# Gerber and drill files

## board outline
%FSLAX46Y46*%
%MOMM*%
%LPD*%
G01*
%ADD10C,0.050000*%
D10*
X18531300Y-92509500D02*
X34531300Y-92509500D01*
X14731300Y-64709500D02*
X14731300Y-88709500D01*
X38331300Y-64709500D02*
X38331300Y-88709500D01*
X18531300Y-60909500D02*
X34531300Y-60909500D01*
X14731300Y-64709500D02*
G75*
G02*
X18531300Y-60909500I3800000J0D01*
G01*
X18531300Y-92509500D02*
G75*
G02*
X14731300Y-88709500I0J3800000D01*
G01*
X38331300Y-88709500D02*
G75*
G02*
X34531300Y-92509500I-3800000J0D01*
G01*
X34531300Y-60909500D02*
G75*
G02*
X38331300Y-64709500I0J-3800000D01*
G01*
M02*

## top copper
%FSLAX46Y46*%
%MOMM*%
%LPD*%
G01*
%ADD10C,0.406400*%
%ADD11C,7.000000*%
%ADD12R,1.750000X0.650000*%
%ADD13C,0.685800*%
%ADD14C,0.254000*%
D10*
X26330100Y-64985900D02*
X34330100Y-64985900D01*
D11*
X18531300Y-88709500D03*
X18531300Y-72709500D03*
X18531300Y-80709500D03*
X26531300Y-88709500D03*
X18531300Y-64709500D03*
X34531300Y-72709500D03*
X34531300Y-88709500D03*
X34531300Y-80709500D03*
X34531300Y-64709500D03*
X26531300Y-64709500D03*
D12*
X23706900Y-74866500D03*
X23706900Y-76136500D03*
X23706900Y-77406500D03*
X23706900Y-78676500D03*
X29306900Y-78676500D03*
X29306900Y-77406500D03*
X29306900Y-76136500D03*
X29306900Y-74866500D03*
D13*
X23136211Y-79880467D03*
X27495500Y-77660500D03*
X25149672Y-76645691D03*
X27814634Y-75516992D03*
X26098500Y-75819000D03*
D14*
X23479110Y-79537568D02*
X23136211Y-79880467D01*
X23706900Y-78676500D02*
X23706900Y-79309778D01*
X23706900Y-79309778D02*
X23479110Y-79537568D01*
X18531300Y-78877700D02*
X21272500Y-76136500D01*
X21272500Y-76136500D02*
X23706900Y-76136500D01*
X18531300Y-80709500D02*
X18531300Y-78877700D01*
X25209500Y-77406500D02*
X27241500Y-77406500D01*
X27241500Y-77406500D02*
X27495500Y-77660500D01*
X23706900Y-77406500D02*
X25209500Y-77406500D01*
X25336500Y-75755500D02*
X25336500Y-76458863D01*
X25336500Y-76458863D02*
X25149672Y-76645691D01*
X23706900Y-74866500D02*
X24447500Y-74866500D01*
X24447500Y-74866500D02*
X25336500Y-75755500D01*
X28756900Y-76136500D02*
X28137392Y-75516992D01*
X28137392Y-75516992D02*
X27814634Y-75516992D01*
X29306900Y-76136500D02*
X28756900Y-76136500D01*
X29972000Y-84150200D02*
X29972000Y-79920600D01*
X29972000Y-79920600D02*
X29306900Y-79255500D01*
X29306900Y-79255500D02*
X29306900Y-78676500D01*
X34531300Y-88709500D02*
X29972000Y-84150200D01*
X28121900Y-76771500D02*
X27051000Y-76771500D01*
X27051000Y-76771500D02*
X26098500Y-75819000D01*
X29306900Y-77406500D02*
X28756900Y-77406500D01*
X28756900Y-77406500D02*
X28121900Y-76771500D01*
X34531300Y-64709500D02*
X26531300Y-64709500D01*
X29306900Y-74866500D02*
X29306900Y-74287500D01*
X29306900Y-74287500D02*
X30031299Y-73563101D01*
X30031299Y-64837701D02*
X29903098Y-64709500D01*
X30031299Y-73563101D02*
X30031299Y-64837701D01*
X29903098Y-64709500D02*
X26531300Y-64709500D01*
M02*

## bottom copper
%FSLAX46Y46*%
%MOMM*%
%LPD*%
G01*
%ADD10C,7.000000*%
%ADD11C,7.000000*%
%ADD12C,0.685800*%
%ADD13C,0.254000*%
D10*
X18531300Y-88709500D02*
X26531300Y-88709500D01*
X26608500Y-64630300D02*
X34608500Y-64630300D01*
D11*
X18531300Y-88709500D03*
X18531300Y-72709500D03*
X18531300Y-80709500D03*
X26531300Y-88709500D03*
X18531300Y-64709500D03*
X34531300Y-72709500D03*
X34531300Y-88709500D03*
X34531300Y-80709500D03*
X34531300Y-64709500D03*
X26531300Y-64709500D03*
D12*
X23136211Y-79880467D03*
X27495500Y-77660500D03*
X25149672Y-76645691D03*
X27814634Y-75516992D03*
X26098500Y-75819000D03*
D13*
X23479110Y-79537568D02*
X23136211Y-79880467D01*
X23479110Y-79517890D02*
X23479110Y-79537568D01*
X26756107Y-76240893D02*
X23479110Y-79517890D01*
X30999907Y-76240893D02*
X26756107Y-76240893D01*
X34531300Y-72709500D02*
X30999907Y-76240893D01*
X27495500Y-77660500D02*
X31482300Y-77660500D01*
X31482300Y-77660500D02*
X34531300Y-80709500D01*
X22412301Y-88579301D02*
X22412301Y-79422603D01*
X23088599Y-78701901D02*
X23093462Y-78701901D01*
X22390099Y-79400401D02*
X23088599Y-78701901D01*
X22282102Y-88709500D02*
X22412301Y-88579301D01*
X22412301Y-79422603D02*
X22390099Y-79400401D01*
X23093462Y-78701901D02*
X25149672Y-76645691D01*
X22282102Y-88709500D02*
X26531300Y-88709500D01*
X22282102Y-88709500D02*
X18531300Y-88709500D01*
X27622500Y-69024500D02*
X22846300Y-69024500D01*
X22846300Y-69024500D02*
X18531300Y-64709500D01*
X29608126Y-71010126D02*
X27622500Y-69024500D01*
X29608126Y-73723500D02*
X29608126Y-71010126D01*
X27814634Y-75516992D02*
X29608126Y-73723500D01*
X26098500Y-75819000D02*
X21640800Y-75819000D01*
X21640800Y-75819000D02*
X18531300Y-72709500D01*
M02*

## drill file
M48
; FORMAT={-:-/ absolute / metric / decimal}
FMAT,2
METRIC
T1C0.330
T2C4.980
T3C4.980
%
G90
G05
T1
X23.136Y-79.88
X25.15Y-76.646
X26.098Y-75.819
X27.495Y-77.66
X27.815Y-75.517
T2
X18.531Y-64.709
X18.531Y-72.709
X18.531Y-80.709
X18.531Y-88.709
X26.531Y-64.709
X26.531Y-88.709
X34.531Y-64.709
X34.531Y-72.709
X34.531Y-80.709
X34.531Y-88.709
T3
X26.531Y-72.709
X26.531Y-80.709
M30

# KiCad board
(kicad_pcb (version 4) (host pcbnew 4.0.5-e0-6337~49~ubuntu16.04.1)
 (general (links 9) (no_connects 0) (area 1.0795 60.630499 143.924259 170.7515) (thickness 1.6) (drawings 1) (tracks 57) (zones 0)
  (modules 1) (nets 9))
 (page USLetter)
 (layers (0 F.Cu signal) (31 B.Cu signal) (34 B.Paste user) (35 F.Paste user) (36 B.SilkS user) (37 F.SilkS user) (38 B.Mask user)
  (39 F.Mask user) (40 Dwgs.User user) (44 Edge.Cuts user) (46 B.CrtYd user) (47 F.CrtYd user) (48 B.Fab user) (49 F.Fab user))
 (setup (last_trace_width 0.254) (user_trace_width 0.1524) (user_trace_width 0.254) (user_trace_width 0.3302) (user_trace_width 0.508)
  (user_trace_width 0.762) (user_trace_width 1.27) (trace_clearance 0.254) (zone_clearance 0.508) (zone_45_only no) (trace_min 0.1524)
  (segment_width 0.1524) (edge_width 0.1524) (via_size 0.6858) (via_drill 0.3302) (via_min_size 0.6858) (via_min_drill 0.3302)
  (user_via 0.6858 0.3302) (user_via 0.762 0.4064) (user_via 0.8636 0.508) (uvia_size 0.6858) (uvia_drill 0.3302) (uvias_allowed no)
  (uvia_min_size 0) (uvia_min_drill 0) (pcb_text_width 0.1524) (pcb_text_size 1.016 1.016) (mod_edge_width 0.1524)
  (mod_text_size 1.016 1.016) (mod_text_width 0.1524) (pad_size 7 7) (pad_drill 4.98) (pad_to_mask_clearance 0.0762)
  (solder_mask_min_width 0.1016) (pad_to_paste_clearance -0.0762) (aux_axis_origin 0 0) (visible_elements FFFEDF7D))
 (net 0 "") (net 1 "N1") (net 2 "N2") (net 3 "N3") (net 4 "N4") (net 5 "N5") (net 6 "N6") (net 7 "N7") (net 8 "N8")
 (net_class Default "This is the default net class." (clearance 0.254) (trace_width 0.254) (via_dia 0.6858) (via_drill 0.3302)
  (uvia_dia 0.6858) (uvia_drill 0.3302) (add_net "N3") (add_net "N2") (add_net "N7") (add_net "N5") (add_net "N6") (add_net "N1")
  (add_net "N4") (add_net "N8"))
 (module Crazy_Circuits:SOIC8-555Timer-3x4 (layer F.Cu) (at 18.5313 88.7095)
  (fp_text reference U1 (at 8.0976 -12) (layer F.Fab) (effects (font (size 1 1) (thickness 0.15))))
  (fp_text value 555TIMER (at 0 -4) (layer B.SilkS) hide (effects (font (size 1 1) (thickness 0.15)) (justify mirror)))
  (fp_line (start 0 0) (end 8 0) (layer B.Cu) (width 7))
  (fp_line (start 0 3.8) (end 16 3.8) (layer Edge.Cuts) (width 0.05))
  (fp_line (start -3.8 -24) (end -3.8 0) (layer Edge.Cuts) (width 0.05))
  (fp_line (start 19.8 -24) (end 19.8 0) (layer Edge.Cuts) (width 0.05))
  (fp_line (start 0 -27.8) (end 16 -27.8) (layer Edge.Cuts) (width 0.05))
  (fp_arc (start 0 -24) (end -3.8 -24) (angle 90) (layer Edge.Cuts) (width 0.05))
  (fp_arc (start 0 0) (end 0 3.8) (angle 90) (layer Edge.Cuts) (width 0.05))
  (fp_arc (start 16 0) (end 19.8 0) (angle 90) (layer Edge.Cuts) (width 0.05))
  (fp_arc (start 16 -24) (end 16 -27.8) (angle 90) (layer Edge.Cuts) (width 0.05))
  (fp_line (start 7.7988 -23.7236) (end 15.7988 -23.7236) (layer F.Cu) (width 0.4064))
  (fp_line (start 8.0772 -24.0792) (end 16.0772 -24.0792) (layer B.Cu) (width 7))
  (pad e thru_hole circle (at 0 0 270) (size 7 7) (drill 4.98) (layers *.Cu *.Mask))
  (pad "" np_thru_hole circle (at 8 -16 270) (size 4.98 4.98) (drill 4.98) (layers *.Cu))
  (pad 6 thru_hole circle (at 0 -16 270) (size 7 7) (drill 4.98) (layers *.Cu B.Mask) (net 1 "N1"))
  (pad 2 thru_hole circle (at 0 -8 270) (size 7 7) (drill 4.98) (layers *.Cu B.Mask) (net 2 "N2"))
  (pad "" np_thru_hole circle (at 8 -8 270) (size 4.98 4.98) (drill 4.98) (layers *.Cu))
  (pad 1 thru_hole circle (at 8 0 270) (size 7 7) (drill 4.98) (layers *.Cu *.Mask) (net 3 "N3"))
  (pad 7 thru_hole circle (at 0 -24 270) (size 7 7) (drill 4.98) (layers *.Cu B.Mask) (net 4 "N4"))
  (pad 4 thru_hole circle (at 16 -16 270) (size 7 7) (drill 4.98) (layers *.Cu B.Mask) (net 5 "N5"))
  (pad 5 thru_hole circle (at 16 0 270) (size 7 7) (drill 4.98) (layers *.Cu B.Mask) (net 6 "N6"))
  (pad 3 thru_hole circle (at 16 -8 270) (size 7 7) (drill 4.98) (layers *.Cu B.Mask) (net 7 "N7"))
  (pad 8 thru_hole circle (at 16 -24 270) (size 7 7) (drill 4.98) (layers *.Cu *.Mask) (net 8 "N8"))
  (pad 8 thru_hole circle (at 8 -24 270) (size 7 7) (drill 4.98) (layers *.Cu *.Mask) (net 8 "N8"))
  (pad 1 smd rect (at 5.1756 -13.843) (size 1.75 0.65) (layers F.Cu F.Paste F.Mask) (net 3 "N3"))
  (pad 2 smd rect (at 5.1756 -12.573) (size 1.75 0.65) (layers F.Cu F.Paste F.Mask) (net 2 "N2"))
  (pad 3 smd rect (at 5.1756 -11.303) (size 1.75 0.65) (layers F.Cu F.Paste F.Mask) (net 7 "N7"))
  (pad 4 smd rect (at 5.1756 -10.033) (size 1.75 0.65) (layers F.Cu F.Paste F.Mask) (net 5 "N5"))
  (pad 5 smd rect (at 10.7756 -10.033) (size 1.75 0.65) (layers F.Cu F.Paste F.Mask) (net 6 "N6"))
  (pad 6 smd rect (at 10.7756 -11.303) (size 1.75 0.65) (layers F.Cu F.Paste F.Mask) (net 1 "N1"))
  (pad 7 smd rect (at 10.7756 -12.573) (size 1.75 0.65) (layers F.Cu F.Paste F.Mask) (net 4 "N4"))
  (pad 8 smd rect (at 10.7756 -13.843) (size 1.75 0.65) (layers F.Cu F.Paste F.Mask) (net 8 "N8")))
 (segment (start 23.47911 79.537568) (end 23.136211 79.880467) (width 0.254) (layer B.Cu) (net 5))
 (segment (start 23.47911 79.51789) (end 23.47911 79.537568) (width 0.254) (layer B.Cu) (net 5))
 (segment (start 26.756107 76.240893) (end 23.47911 79.51789) (width 0.254) (layer B.Cu) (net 5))
 (segment (start 30.999907 76.240893) (end 26.756107 76.240893) (width 0.254) (layer B.Cu) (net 5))
 (segment (start 34.5313 72.7095) (end 30.999907 76.240893) (width 0.254) (layer B.Cu) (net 5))
 (segment (start 23.47911 79.537568) (end 23.136211 79.880467) (width 0.254) (layer F.Cu) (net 5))
 (segment (start 23.7069 78.6765) (end 23.7069 79.309778) (width 0.254) (layer F.Cu) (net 5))
 (segment (start 23.7069 79.309778) (end 23.47911 79.537568) (width 0.254) (layer F.Cu) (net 5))
 (via (at 23.136211 79.880467) (size 0.6858) (drill 0.3302) (layers F.Cu B.Cu) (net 5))
 (segment (start 18.5313 78.8777) (end 21.2725 76.1365) (width 0.254) (layer F.Cu) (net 2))
 (segment (start 21.2725 76.1365) (end 23.7069 76.1365) (width 0.254) (layer F.Cu) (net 2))
 (segment (start 18.5313 80.7095) (end 18.5313 78.8777) (width 0.254) (layer F.Cu) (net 2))
 (segment (start 27.4955 77.6605) (end 31.4823 77.6605) (width 0.254) (layer B.Cu) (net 7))
 (segment (start 31.4823 77.6605) (end 34.5313 80.7095) (width 0.254) (layer B.Cu) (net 7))
 (segment (start 25.2095 77.4065) (end 27.2415 77.4065) (width 0.254) (layer F.Cu) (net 7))
 (segment (start 27.2415 77.4065) (end 27.4955 77.6605) (width 0.254) (layer F.Cu) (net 7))
 (via (at 27.4955 77.6605) (size 0.6858) (drill 0.3302) (layers F.Cu B.Cu) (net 7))
 (segment (start 23.7069 77.4065) (end 25.2095 77.4065) (width 0.254) (layer F.Cu) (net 7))
 (segment (start 22.412301 88.579301) (end 22.412301 79.422603) (width 0.254) (layer B.Cu) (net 3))
 (segment (start 23.088599 78.701901) (end 23.093462 78.701901) (width 0.254) (layer B.Cu) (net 3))
 (segment (start 22.390099 79.400401) (end 23.088599 78.701901) (width 0.254) (layer B.Cu) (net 3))
 (segment (start 22.282102 88.7095) (end 22.412301 88.579301) (width 0.254) (layer B.Cu) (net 3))
 (segment (start 22.412301 79.422603) (end 22.390099 79.400401) (width 0.254) (layer B.Cu) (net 3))
 (segment (start 23.093462 78.701901) (end 25.149672 76.645691) (width 0.254) (layer B.Cu) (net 3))
 (segment (start 25.3365 75.7555) (end 25.3365 76.458863) (width 0.254) (layer F.Cu) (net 3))
 (segment (start 25.3365 76.458863) (end 25.149672 76.645691) (width 0.254) (layer F.Cu) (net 3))
 (via (at 25.149672 76.645691) (size 0.6858) (drill 0.3302) (layers F.Cu B.Cu) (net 3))
 (segment (start 22.282102 88.7095) (end 26.5313 88.7095) (width 0.254) (layer B.Cu) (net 3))
 (segment (start 22.282102 88.7095) (end 18.5313 88.7095) (width 0.254) (layer B.Cu) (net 3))
 (segment (start 23.7069 74.8665) (end 24.4475 74.8665) (width 0.254) (layer F.Cu) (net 3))
 (segment (start 24.4475 74.8665) (end 25.3365 75.7555) (width 0.254) (layer F.Cu) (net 3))
 (segment (start 27.6225 69.0245) (end 22.8463 69.0245) (width 0.254) (layer B.Cu) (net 4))
 (segment (start 22.8463 69.0245) (end 18.5313 64.7095) (width 0.254) (layer B.Cu) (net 4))
 (segment (start 29.608126 71.010126) (end 27.6225 69.0245) (width 0.254) (layer B.Cu) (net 4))
 (segment (start 29.608126 73.7235) (end 29.608126 71.010126) (width 0.254) (layer B.Cu) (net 4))
 (segment (start 27.814634 75.516992) (end 29.608126 73.7235) (width 0.254) (layer B.Cu) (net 4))
 (segment (start 28.7569 76.1365) (end 28.137392 75.516992) (width 0.254) (layer F.Cu) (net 4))
 (segment (start 28.137392 75.516992) (end 27.814634 75.516992) (width 0.254) (layer F.Cu) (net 4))
 (via (at 27.814634 75.516992) (size 0.6858) (drill 0.3302) (layers F.Cu B.Cu) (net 4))
 (segment (start 29.3069 76.1365) (end 28.7569 76.1365) (width 0.254) (layer F.Cu) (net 4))
 (segment (start 29.972 84.1502) (end 29.972 79.9206) (width 0.254) (layer F.Cu) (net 6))
 (segment (start 29.972 79.9206) (end 29.3069 79.2555) (width 0.254) (layer F.Cu) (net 6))
 (segment (start 29.3069 79.2555) (end 29.3069 78.6765) (width 0.254) (layer F.Cu) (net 6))
 (segment (start 34.5313 88.7095) (end 29.972 84.1502) (width 0.254) (layer F.Cu) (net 6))
 (segment (start 26.0985 75.819) (end 21.6408 75.819) (width 0.254) (layer B.Cu) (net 1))
 (segment (start 21.6408 75.819) (end 18.5313 72.7095) (width 0.254) (layer B.Cu) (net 1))
 (segment (start 28.1219 76.7715) (end 27.051 76.7715) (width 0.254) (layer F.Cu) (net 1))
 (segment (start 27.051 76.7715) (end 26.0985 75.819) (width 0.254) (layer F.Cu) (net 1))
 (via (at 26.0985 75.819) (size 0.6858) (drill 0.3302) (layers F.Cu B.Cu) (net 1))
 (segment (start 29.3069 77.4065) (end 28.7569 77.4065) (width 0.254) (layer F.Cu) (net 1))
 (segment (start 28.7569 77.4065) (end 28.1219 76.7715) (width 0.254) (layer F.Cu) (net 1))
 (segment (start 34.5313 64.7095) (end 26.5313 64.7095) (width 0.254) (layer F.Cu) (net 8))
 (segment (start 29.3069 74.8665) (end 29.3069 74.2875) (width 0.254) (layer F.Cu) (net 8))
 (segment (start 29.3069 74.2875) (end 30.031299 73.563101) (width 0.254) (layer F.Cu) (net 8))
 (segment (start 30.031299 64.837701) (end 29.903098 64.7095) (width 0.254) (layer F.Cu) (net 8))
 (segment (start 30.031299 73.563101) (end 30.031299 64.837701) (width 0.254) (layer F.Cu) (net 8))
 (segment (start 29.903098 64.7095) (end 26.5313 64.7095) (width 0.254) (layer F.Cu) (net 8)))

